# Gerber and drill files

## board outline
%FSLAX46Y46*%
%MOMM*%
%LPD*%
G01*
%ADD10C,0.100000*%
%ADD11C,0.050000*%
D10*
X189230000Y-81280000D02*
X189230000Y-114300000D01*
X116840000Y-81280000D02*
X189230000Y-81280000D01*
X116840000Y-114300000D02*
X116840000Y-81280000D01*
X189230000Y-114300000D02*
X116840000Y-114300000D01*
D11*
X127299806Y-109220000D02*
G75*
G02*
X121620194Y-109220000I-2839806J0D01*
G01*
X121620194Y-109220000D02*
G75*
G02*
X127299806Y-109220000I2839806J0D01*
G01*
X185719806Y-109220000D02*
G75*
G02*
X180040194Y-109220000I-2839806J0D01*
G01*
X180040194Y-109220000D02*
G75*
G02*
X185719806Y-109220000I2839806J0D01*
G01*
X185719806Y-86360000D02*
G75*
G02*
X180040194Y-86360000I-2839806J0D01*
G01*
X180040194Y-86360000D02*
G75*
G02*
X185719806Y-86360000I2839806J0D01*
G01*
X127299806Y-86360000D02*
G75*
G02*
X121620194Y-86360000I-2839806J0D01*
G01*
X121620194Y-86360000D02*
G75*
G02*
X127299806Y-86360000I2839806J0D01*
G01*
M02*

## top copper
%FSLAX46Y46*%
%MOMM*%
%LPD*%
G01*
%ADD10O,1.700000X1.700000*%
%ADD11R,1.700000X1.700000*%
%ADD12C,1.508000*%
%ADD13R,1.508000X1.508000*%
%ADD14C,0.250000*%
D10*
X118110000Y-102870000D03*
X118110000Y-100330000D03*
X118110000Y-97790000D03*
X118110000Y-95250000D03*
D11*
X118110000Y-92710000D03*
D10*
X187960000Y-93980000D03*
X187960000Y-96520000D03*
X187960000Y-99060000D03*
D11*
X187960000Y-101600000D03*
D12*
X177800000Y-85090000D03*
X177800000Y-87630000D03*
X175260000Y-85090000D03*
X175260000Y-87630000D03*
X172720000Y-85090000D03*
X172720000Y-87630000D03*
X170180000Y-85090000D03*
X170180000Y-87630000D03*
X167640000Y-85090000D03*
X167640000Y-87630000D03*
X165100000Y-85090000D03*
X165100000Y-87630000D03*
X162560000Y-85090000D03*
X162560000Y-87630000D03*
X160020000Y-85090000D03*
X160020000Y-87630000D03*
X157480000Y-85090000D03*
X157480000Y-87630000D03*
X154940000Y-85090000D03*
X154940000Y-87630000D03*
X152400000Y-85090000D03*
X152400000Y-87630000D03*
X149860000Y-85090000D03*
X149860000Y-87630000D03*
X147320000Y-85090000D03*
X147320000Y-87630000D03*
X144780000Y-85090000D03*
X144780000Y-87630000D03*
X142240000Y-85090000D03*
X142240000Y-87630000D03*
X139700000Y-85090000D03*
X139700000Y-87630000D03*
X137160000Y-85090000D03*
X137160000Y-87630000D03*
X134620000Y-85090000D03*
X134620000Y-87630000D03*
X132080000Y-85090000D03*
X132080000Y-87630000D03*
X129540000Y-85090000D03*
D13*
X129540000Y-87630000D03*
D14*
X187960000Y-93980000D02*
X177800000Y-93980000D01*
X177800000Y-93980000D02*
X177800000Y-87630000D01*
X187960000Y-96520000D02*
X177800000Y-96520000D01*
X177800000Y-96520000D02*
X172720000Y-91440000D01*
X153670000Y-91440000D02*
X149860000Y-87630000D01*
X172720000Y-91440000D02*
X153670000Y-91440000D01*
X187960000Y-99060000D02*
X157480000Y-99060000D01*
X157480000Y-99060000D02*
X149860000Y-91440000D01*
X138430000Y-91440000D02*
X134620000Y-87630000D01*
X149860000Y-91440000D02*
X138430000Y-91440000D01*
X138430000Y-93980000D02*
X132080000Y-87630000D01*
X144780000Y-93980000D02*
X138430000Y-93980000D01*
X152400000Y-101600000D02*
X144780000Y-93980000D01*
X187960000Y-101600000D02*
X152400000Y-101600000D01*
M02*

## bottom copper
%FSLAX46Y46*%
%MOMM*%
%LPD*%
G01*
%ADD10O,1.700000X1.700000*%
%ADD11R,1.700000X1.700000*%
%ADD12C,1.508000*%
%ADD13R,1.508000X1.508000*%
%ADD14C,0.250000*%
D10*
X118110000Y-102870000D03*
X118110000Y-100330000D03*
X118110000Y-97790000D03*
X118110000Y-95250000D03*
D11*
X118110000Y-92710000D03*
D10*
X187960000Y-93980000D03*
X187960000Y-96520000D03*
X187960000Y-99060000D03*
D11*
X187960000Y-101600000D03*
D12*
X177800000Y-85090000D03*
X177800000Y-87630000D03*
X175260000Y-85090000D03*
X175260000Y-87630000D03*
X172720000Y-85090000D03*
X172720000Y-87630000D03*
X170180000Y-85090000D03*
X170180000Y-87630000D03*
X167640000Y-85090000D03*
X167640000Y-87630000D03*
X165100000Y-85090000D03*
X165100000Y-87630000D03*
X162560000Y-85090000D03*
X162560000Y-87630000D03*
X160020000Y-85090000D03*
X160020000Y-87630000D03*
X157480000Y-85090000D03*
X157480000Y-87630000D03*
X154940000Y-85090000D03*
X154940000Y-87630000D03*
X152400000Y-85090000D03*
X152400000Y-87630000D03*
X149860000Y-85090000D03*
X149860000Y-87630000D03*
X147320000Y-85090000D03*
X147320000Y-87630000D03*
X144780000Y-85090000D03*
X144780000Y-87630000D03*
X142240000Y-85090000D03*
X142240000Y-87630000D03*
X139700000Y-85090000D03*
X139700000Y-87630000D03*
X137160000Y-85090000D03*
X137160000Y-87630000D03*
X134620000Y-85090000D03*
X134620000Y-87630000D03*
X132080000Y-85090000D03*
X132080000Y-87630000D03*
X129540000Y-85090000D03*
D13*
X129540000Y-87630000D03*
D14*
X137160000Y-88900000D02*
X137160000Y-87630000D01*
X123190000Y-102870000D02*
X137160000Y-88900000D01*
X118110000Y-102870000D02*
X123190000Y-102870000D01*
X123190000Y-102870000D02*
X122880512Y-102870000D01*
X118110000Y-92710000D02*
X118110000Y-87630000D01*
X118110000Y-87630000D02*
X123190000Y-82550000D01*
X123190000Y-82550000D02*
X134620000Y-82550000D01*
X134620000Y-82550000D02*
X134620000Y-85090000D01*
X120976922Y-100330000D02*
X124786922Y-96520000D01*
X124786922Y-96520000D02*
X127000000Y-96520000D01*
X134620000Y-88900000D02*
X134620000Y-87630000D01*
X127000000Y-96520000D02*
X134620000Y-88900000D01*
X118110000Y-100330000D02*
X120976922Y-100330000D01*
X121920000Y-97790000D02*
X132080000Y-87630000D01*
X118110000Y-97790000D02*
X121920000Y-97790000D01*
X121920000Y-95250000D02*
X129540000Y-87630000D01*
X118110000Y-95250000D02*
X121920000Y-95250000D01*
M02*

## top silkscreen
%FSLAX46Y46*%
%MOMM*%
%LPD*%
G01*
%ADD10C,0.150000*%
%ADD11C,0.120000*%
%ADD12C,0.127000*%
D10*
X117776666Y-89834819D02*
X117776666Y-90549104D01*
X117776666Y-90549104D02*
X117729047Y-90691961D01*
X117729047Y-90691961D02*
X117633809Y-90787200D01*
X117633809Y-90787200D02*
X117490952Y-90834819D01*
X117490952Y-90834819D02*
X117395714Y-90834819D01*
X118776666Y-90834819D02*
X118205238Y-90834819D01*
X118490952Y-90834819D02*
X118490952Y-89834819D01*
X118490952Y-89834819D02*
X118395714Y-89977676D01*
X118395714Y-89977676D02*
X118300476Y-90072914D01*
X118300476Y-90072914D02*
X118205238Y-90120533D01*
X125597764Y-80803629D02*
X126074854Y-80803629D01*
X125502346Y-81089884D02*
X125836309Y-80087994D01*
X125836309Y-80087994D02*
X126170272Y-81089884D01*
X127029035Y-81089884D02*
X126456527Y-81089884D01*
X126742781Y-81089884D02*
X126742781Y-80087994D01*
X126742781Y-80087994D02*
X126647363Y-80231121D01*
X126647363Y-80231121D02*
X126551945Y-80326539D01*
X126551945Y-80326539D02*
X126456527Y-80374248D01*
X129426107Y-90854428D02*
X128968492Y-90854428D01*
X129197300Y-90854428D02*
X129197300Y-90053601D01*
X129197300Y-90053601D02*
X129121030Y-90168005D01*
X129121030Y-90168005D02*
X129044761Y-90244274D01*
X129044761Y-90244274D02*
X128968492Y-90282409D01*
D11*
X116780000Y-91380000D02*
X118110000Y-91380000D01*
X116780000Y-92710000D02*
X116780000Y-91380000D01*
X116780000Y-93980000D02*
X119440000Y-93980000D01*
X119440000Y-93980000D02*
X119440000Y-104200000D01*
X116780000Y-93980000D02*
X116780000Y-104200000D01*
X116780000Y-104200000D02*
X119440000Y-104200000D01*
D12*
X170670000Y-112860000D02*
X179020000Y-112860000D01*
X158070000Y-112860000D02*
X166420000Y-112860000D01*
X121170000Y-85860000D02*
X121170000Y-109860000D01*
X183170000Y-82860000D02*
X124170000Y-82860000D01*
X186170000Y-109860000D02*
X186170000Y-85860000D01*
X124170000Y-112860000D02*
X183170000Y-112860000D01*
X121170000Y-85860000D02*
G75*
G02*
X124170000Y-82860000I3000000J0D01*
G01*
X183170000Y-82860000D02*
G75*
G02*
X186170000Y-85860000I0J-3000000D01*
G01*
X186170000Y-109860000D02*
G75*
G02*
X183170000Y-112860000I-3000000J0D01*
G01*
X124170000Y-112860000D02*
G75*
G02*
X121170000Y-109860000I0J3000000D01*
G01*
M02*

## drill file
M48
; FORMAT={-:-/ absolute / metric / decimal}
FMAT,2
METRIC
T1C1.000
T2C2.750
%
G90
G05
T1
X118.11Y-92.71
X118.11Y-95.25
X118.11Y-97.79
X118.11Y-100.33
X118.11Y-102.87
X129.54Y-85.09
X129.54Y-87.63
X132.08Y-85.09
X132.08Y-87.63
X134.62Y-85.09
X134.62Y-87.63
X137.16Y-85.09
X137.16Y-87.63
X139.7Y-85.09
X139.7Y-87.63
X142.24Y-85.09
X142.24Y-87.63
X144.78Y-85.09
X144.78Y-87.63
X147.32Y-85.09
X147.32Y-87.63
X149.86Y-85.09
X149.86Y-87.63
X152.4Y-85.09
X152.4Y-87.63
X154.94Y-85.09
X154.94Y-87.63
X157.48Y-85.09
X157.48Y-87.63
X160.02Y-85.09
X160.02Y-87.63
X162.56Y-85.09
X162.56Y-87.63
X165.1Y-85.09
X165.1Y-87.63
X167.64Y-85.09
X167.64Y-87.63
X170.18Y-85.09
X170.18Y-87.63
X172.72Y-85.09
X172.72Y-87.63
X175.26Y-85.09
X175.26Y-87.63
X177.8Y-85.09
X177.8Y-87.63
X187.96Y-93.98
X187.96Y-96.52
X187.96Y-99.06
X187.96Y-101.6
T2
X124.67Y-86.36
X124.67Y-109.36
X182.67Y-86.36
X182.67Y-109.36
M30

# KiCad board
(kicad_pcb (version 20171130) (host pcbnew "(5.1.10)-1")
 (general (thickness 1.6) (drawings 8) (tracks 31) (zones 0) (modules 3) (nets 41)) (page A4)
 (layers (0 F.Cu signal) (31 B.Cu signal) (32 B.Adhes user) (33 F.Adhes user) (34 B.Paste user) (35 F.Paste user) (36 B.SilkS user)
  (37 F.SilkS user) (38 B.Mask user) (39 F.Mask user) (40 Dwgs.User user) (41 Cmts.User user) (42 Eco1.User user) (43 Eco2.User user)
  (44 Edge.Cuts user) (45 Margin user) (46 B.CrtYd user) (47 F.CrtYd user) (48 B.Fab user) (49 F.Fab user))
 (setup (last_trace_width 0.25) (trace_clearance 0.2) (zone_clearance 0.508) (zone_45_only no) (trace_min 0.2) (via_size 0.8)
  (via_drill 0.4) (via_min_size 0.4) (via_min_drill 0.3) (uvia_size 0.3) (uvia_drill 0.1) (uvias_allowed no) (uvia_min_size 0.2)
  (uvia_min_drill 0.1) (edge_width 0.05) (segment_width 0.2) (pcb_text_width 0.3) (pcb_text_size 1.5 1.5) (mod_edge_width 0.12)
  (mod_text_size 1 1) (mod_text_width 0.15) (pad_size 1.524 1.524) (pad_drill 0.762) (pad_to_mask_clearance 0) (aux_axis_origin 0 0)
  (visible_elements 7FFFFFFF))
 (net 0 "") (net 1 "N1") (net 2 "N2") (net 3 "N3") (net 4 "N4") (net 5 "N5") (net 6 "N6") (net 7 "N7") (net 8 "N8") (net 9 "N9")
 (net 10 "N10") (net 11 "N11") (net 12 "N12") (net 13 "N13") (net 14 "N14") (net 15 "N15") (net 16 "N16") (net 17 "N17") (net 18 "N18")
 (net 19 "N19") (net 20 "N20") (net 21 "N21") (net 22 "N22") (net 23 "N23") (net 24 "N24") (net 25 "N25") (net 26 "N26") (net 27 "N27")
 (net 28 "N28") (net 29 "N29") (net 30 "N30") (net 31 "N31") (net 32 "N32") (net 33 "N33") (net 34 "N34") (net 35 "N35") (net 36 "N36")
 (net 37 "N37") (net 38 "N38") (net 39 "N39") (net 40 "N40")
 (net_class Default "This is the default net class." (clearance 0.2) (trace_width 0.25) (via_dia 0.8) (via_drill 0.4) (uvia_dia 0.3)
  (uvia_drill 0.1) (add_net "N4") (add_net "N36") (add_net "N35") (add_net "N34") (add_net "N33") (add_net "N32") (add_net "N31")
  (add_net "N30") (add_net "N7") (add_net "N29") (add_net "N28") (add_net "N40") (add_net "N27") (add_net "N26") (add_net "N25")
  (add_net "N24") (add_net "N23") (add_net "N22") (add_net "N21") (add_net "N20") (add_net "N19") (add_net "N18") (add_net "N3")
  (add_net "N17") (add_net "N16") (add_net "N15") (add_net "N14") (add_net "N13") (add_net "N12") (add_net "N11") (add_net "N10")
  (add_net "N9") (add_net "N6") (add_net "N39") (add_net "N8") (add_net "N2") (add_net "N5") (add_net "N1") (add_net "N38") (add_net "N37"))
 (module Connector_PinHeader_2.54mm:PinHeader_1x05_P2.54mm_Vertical (layer F.Cu) (at 118.11 92.71)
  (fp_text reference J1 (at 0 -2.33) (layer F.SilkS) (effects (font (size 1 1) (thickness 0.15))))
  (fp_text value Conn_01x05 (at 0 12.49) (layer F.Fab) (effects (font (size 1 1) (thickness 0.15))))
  (fp_line (start -1.33 -1.33) (end 0 -1.33) (layer F.SilkS) (width 0.12))
  (fp_line (start -1.33 0) (end -1.33 -1.33) (layer F.SilkS) (width 0.12))
  (fp_line (start -1.33 1.27) (end 1.33 1.27) (layer F.SilkS) (width 0.12))
  (fp_line (start 1.33 1.27) (end 1.33 11.49) (layer F.SilkS) (width 0.12))
  (fp_line (start -1.33 1.27) (end -1.33 11.49) (layer F.SilkS) (width 0.12))
  (fp_line (start -1.33 11.49) (end 1.33 11.49) (layer F.SilkS) (width 0.12))
  (pad 5 thru_hole oval (at 0 10.16) (size 1.7 1.7) (drill 1) (layers *.Cu *.Mask) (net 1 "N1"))
  (pad 4 thru_hole oval (at 0 7.62) (size 1.7 1.7) (drill 1) (layers *.Cu *.Mask) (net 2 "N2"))
  (pad 3 thru_hole oval (at 0 5.08) (size 1.7 1.7) (drill 1) (layers *.Cu *.Mask) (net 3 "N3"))
  (pad 2 thru_hole oval (at 0 2.54) (size 1.7 1.7) (drill 1) (layers *.Cu *.Mask) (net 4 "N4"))
  (pad 1 thru_hole rect (at 0 0) (size 1.7 1.7) (drill 1) (layers *.Cu *.Mask) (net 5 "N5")))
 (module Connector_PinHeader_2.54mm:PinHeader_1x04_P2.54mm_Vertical (layer B.Cu) (at 187.96 101.6)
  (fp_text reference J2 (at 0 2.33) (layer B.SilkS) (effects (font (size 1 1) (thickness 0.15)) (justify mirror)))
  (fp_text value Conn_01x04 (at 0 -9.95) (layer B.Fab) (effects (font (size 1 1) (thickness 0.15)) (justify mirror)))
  (pad 4 thru_hole oval (at 0 -7.62) (size 1.7 1.7) (drill 1) (layers *.Cu *.Mask) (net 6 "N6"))
  (pad 3 thru_hole oval (at 0 -5.08) (size 1.7 1.7) (drill 1) (layers *.Cu *.Mask) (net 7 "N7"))
  (pad 2 thru_hole oval (at 0 -2.54) (size 1.7 1.7) (drill 1) (layers *.Cu *.Mask) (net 2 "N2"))
  (pad 1 thru_hole rect (at 0 0) (size 1.7 1.7) (drill 1) (layers *.Cu *.Mask) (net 3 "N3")))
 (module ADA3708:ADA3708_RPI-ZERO (layer F.Cu) (at 153.67 86.36)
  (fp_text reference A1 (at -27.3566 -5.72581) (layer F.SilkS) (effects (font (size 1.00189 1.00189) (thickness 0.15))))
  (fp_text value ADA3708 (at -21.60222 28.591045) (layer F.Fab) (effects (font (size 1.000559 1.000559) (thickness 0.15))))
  (fp_line (start 17 26.5) (end 25.35 26.5) (layer F.SilkS) (width 0.127))
  (fp_line (start 4.4 26.5) (end 12.75 26.5) (layer F.SilkS) (width 0.127))
  (fp_line (start -32.5 -0.5) (end -32.5 23.5) (layer F.SilkS) (width 0.127))
  (fp_line (start 29.5 -3.5) (end -29.5 -3.5) (layer F.SilkS) (width 0.127))
  (fp_line (start 32.5 23.5) (end 32.5 -0.5) (layer F.SilkS) (width 0.127))
  (fp_line (start -29.5 26.5) (end 29.5 26.5) (layer F.SilkS) (width 0.127))
  (fp_arc (start -29.5 -0.5) (end -32.5 -0.5) (angle 90) (layer F.SilkS) (width 0.127))
  (fp_arc (start 29.5 -0.5) (end 29.5 -3.5) (angle 90) (layer F.SilkS) (width 0.127))
  (fp_arc (start 29.5 23.5) (end 32.5 23.5) (angle 90) (layer F.SilkS) (width 0.127))
  (fp_arc (start -29.5 23.5) (end -29.5 26.5) (angle 90) (layer F.SilkS) (width 0.127))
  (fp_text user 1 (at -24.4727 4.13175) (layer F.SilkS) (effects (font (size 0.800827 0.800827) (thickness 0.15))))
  (pad None np_thru_hole circle (at 29 0) (size 2.75 2.75) (drill 2.75) (layers *.Cu *.Mask))
  (pad None np_thru_hole circle (at 29 23) (size 2.75 2.75) (drill 2.75) (layers *.Cu *.Mask))
  (pad None np_thru_hole circle (at -29 0) (size 2.75 2.75) (drill 2.75) (layers *.Cu *.Mask))
  (pad None np_thru_hole circle (at -29 23) (size 2.75 2.75) (drill 2.75) (layers *.Cu *.Mask))
  (pad 40 thru_hole circle (at 24.13 -1.27) (size 1.508 1.508) (drill 1) (layers *.Cu *.Mask) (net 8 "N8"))
  (pad 39 thru_hole circle (at 24.13 1.27) (size 1.508 1.508) (drill 1) (layers *.Cu *.Mask) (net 6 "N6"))
  (pad 38 thru_hole circle (at 21.59 -1.27) (size 1.508 1.508) (drill 1) (layers *.Cu *.Mask) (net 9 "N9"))
  (pad 37 thru_hole circle (at 21.59 1.27) (size 1.508 1.508) (drill 1) (layers *.Cu *.Mask) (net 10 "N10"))
  (pad 36 thru_hole circle (at 19.05 -1.27) (size 1.508 1.508) (drill 1) (layers *.Cu *.Mask) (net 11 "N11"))
  (pad 35 thru_hole circle (at 19.05 1.27) (size 1.508 1.508) (drill 1) (layers *.Cu *.Mask) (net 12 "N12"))
  (pad 34 thru_hole circle (at 16.51 -1.27) (size 1.508 1.508) (drill 1) (layers *.Cu *.Mask) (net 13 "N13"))
  (pad 33 thru_hole circle (at 16.51 1.27) (size 1.508 1.508) (drill 1) (layers *.Cu *.Mask) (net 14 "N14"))
  (pad 32 thru_hole circle (at 13.97 -1.27) (size 1.508 1.508) (drill 1) (layers *.Cu *.Mask) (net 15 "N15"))
  (pad 31 thru_hole circle (at 13.97 1.27) (size 1.508 1.508) (drill 1) (layers *.Cu *.Mask) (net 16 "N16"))
  (pad 30 thru_hole circle (at 11.43 -1.27) (size 1.508 1.508) (drill 1) (layers *.Cu *.Mask) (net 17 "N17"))
  (pad 29 thru_hole circle (at 11.43 1.27) (size 1.508 1.508) (drill 1) (layers *.Cu *.Mask) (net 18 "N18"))
  (pad 28 thru_hole circle (at 8.89 -1.27) (size 1.508 1.508) (drill 1) (layers *.Cu *.Mask) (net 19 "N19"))
  (pad 27 thru_hole circle (at 8.89 1.27) (size 1.508 1.508) (drill 1) (layers *.Cu *.Mask) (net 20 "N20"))
  (pad 26 thru_hole circle (at 6.35 -1.27) (size 1.508 1.508) (drill 1) (layers *.Cu *.Mask) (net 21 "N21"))
  (pad 25 thru_hole circle (at 6.35 1.27) (size 1.508 1.508) (drill 1) (layers *.Cu *.Mask) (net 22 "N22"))
  (pad 24 thru_hole circle (at 3.81 -1.27) (size 1.508 1.508) (drill 1) (layers *.Cu *.Mask) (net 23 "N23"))
  (pad 23 thru_hole circle (at 3.81 1.27) (size 1.508 1.508) (drill 1) (layers *.Cu *.Mask) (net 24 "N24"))
  (pad 22 thru_hole circle (at 1.27 -1.27) (size 1.508 1.508) (drill 1) (layers *.Cu *.Mask) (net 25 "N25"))
  (pad 21 thru_hole circle (at 1.27 1.27) (size 1.508 1.508) (drill 1) (layers *.Cu *.Mask) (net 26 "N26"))
  (pad 20 thru_hole circle (at -1.27 -1.27) (size 1.508 1.508) (drill 1) (layers *.Cu *.Mask) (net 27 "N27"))
  (pad 19 thru_hole circle (at -1.27 1.27) (size 1.508 1.508) (drill 1) (layers *.Cu *.Mask) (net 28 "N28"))
  (pad 18 thru_hole circle (at -3.81 -1.27) (size 1.508 1.508) (drill 1) (layers *.Cu *.Mask) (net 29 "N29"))
  (pad 17 thru_hole circle (at -3.81 1.27) (size 1.508 1.508) (drill 1) (layers *.Cu *.Mask) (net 7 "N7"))
  (pad 16 thru_hole circle (at -6.35 -1.27) (size 1.508 1.508) (drill 1) (layers *.Cu *.Mask) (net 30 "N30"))
  (pad 15 thru_hole circle (at -6.35 1.27) (size 1.508 1.508) (drill 1) (layers *.Cu *.Mask) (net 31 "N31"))
  (pad 14 thru_hole circle (at -8.89 -1.27) (size 1.508 1.508) (drill 1) (layers *.Cu *.Mask) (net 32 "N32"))
  (pad 13 thru_hole circle (at -8.89 1.27) (size 1.508 1.508) (drill 1) (layers *.Cu *.Mask) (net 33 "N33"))
  (pad 12 thru_hole circle (at -11.43 -1.27) (size 1.508 1.508) (drill 1) (layers *.Cu *.Mask) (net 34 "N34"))
  (pad 11 thru_hole circle (at -11.43 1.27) (size 1.508 1.508) (drill 1) (layers *.Cu *.Mask) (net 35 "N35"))
  (pad 10 thru_hole circle (at -13.97 -1.27) (size 1.508 1.508) (drill 1) (layers *.Cu *.Mask) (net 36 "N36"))
  (pad 9 thru_hole circle (at -13.97 1.27) (size 1.508 1.508) (drill 1) (layers *.Cu *.Mask) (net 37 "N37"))
  (pad 8 thru_hole circle (at -16.51 -1.27) (size 1.508 1.508) (drill 1) (layers *.Cu *.Mask) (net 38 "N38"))
  (pad 7 thru_hole circle (at -16.51 1.27) (size 1.508 1.508) (drill 1) (layers *.Cu *.Mask) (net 1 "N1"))
  (pad 6 thru_hole circle (at -19.05 -1.27) (size 1.508 1.508) (drill 1) (layers *.Cu *.Mask) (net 5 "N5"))
  (pad 5 thru_hole circle (at -19.05 1.27) (size 1.508 1.508) (drill 1) (layers *.Cu *.Mask) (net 2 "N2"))
  (pad 4 thru_hole circle (at -21.59 -1.27) (size 1.508 1.508) (drill 1) (layers *.Cu *.Mask) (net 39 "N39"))
  (pad 3 thru_hole circle (at -21.59 1.27) (size 1.508 1.508) (drill 1) (layers *.Cu *.Mask) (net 3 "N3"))
  (pad 2 thru_hole circle (at -24.13 -1.27) (size 1.508 1.508) (drill 1) (layers *.Cu *.Mask) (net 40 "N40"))
  (pad 1 thru_hole rect (at -24.13 1.27) (size 1.508 1.508) (drill 1) (layers *.Cu *.Mask) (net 4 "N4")))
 (gr_line (start 189.23 81.28) (end 189.23 114.3) (layer Edge.Cuts) (width 0.1))
 (gr_line (start 116.84 81.28) (end 189.23 81.28) (layer Edge.Cuts) (width 0.1))
 (gr_line (start 116.84 114.3) (end 116.84 81.28) (layer Edge.Cuts) (width 0.1))
 (gr_line (start 189.23 114.3) (end 116.84 114.3) (layer Edge.Cuts) (width 0.1))
 (gr_circle (center 124.46 109.22) (end 127 110.49) (layer Edge.Cuts) (width 0.05))
 (gr_circle (center 182.88 109.22) (end 185.42 110.49) (layer Edge.Cuts) (width 0.05))
 (gr_circle (center 182.88 86.36) (end 185.42 87.63) (layer Edge.Cuts) (width 0.05))
 (gr_circle (center 124.46 86.36) (end 127 87.63) (layer Edge.Cuts) (width 0.05))
 (segment (start 187.96 93.98) (end 177.8 93.98) (width 0.25) (layer F.Cu) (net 6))
 (segment (start 177.8 93.98) (end 177.8 87.63) (width 0.25) (layer F.Cu) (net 6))
 (segment (start 187.96 96.52) (end 177.8 96.52) (width 0.25) (layer F.Cu) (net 7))
 (segment (start 177.8 96.52) (end 172.72 91.44) (width 0.25) (layer F.Cu) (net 7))
 (segment (start 153.67 91.44) (end 149.86 87.63) (width 0.25) (layer F.Cu) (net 7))
 (segment (start 172.72 91.44) (end 153.67 91.44) (width 0.25) (layer F.Cu) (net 7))
 (segment (start 137.16 88.9) (end 137.16 87.63) (width 0.25) (layer B.Cu) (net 1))
 (segment (start 123.19 102.87) (end 137.16 88.9) (width 0.25) (layer B.Cu) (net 1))
 (segment (start 118.11 102.87) (end 123.19 102.87) (width 0.25) (layer B.Cu) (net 1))
 (segment (start 123.19 102.87) (end 122.880512 102.87) (width 0.25) (layer B.Cu) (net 1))
 (segment (start 118.11 92.71) (end 118.11 87.63) (width 0.25) (layer B.Cu) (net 5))
 (segment (start 118.11 87.63) (end 123.19 82.55) (width 0.25) (layer B.Cu) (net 5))
 (segment (start 123.19 82.55) (end 134.62 82.55) (width 0.25) (layer B.Cu) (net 5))
 (segment (start 134.62 82.55) (end 134.62 85.09) (width 0.25) (layer B.Cu) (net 5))
 (segment (start 187.96 99.06) (end 157.48 99.06) (width 0.25) (layer F.Cu) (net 2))
 (segment (start 157.48 99.06) (end 149.86 91.44) (width 0.25) (layer F.Cu) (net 2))
 (segment (start 138.43 91.44) (end 134.62 87.63) (width 0.25) (layer F.Cu) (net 2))
 (segment (start 149.86 91.44) (end 138.43 91.44) (width 0.25) (layer F.Cu) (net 2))
 (segment (start 120.976922 100.33) (end 124.786922 96.52) (width 0.25) (layer B.Cu) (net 2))
 (segment (start 124.786922 96.52) (end 127 96.52) (width 0.25) (layer B.Cu) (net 2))
 (segment (start 134.62 88.9) (end 134.62 87.63) (width 0.25) (layer B.Cu) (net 2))
 (segment (start 127 96.52) (end 134.62 88.9) (width 0.25) (layer B.Cu) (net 2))
 (segment (start 118.11 100.33) (end 120.976922 100.33) (width 0.25) (layer B.Cu) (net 2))
 (segment (start 138.43 93.98) (end 132.08 87.63) (width 0.25) (layer F.Cu) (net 3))
 (segment (start 144.78 93.98) (end 138.43 93.98) (width 0.25) (layer F.Cu) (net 3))
 (segment (start 152.4 101.6) (end 144.78 93.98) (width 0.25) (layer F.Cu) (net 3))
 (segment (start 187.96 101.6) (end 152.4 101.6) (width 0.25) (layer F.Cu) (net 3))
 (segment (start 121.92 97.79) (end 132.08 87.63) (width 0.25) (layer B.Cu) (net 3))
 (segment (start 118.11 97.79) (end 121.92 97.79) (width 0.25) (layer B.Cu) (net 3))
 (segment (start 121.92 95.25) (end 129.54 87.63) (width 0.25) (layer B.Cu) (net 4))
 (segment (start 118.11 95.25) (end 121.92 95.25) (width 0.25) (layer B.Cu) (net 4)))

